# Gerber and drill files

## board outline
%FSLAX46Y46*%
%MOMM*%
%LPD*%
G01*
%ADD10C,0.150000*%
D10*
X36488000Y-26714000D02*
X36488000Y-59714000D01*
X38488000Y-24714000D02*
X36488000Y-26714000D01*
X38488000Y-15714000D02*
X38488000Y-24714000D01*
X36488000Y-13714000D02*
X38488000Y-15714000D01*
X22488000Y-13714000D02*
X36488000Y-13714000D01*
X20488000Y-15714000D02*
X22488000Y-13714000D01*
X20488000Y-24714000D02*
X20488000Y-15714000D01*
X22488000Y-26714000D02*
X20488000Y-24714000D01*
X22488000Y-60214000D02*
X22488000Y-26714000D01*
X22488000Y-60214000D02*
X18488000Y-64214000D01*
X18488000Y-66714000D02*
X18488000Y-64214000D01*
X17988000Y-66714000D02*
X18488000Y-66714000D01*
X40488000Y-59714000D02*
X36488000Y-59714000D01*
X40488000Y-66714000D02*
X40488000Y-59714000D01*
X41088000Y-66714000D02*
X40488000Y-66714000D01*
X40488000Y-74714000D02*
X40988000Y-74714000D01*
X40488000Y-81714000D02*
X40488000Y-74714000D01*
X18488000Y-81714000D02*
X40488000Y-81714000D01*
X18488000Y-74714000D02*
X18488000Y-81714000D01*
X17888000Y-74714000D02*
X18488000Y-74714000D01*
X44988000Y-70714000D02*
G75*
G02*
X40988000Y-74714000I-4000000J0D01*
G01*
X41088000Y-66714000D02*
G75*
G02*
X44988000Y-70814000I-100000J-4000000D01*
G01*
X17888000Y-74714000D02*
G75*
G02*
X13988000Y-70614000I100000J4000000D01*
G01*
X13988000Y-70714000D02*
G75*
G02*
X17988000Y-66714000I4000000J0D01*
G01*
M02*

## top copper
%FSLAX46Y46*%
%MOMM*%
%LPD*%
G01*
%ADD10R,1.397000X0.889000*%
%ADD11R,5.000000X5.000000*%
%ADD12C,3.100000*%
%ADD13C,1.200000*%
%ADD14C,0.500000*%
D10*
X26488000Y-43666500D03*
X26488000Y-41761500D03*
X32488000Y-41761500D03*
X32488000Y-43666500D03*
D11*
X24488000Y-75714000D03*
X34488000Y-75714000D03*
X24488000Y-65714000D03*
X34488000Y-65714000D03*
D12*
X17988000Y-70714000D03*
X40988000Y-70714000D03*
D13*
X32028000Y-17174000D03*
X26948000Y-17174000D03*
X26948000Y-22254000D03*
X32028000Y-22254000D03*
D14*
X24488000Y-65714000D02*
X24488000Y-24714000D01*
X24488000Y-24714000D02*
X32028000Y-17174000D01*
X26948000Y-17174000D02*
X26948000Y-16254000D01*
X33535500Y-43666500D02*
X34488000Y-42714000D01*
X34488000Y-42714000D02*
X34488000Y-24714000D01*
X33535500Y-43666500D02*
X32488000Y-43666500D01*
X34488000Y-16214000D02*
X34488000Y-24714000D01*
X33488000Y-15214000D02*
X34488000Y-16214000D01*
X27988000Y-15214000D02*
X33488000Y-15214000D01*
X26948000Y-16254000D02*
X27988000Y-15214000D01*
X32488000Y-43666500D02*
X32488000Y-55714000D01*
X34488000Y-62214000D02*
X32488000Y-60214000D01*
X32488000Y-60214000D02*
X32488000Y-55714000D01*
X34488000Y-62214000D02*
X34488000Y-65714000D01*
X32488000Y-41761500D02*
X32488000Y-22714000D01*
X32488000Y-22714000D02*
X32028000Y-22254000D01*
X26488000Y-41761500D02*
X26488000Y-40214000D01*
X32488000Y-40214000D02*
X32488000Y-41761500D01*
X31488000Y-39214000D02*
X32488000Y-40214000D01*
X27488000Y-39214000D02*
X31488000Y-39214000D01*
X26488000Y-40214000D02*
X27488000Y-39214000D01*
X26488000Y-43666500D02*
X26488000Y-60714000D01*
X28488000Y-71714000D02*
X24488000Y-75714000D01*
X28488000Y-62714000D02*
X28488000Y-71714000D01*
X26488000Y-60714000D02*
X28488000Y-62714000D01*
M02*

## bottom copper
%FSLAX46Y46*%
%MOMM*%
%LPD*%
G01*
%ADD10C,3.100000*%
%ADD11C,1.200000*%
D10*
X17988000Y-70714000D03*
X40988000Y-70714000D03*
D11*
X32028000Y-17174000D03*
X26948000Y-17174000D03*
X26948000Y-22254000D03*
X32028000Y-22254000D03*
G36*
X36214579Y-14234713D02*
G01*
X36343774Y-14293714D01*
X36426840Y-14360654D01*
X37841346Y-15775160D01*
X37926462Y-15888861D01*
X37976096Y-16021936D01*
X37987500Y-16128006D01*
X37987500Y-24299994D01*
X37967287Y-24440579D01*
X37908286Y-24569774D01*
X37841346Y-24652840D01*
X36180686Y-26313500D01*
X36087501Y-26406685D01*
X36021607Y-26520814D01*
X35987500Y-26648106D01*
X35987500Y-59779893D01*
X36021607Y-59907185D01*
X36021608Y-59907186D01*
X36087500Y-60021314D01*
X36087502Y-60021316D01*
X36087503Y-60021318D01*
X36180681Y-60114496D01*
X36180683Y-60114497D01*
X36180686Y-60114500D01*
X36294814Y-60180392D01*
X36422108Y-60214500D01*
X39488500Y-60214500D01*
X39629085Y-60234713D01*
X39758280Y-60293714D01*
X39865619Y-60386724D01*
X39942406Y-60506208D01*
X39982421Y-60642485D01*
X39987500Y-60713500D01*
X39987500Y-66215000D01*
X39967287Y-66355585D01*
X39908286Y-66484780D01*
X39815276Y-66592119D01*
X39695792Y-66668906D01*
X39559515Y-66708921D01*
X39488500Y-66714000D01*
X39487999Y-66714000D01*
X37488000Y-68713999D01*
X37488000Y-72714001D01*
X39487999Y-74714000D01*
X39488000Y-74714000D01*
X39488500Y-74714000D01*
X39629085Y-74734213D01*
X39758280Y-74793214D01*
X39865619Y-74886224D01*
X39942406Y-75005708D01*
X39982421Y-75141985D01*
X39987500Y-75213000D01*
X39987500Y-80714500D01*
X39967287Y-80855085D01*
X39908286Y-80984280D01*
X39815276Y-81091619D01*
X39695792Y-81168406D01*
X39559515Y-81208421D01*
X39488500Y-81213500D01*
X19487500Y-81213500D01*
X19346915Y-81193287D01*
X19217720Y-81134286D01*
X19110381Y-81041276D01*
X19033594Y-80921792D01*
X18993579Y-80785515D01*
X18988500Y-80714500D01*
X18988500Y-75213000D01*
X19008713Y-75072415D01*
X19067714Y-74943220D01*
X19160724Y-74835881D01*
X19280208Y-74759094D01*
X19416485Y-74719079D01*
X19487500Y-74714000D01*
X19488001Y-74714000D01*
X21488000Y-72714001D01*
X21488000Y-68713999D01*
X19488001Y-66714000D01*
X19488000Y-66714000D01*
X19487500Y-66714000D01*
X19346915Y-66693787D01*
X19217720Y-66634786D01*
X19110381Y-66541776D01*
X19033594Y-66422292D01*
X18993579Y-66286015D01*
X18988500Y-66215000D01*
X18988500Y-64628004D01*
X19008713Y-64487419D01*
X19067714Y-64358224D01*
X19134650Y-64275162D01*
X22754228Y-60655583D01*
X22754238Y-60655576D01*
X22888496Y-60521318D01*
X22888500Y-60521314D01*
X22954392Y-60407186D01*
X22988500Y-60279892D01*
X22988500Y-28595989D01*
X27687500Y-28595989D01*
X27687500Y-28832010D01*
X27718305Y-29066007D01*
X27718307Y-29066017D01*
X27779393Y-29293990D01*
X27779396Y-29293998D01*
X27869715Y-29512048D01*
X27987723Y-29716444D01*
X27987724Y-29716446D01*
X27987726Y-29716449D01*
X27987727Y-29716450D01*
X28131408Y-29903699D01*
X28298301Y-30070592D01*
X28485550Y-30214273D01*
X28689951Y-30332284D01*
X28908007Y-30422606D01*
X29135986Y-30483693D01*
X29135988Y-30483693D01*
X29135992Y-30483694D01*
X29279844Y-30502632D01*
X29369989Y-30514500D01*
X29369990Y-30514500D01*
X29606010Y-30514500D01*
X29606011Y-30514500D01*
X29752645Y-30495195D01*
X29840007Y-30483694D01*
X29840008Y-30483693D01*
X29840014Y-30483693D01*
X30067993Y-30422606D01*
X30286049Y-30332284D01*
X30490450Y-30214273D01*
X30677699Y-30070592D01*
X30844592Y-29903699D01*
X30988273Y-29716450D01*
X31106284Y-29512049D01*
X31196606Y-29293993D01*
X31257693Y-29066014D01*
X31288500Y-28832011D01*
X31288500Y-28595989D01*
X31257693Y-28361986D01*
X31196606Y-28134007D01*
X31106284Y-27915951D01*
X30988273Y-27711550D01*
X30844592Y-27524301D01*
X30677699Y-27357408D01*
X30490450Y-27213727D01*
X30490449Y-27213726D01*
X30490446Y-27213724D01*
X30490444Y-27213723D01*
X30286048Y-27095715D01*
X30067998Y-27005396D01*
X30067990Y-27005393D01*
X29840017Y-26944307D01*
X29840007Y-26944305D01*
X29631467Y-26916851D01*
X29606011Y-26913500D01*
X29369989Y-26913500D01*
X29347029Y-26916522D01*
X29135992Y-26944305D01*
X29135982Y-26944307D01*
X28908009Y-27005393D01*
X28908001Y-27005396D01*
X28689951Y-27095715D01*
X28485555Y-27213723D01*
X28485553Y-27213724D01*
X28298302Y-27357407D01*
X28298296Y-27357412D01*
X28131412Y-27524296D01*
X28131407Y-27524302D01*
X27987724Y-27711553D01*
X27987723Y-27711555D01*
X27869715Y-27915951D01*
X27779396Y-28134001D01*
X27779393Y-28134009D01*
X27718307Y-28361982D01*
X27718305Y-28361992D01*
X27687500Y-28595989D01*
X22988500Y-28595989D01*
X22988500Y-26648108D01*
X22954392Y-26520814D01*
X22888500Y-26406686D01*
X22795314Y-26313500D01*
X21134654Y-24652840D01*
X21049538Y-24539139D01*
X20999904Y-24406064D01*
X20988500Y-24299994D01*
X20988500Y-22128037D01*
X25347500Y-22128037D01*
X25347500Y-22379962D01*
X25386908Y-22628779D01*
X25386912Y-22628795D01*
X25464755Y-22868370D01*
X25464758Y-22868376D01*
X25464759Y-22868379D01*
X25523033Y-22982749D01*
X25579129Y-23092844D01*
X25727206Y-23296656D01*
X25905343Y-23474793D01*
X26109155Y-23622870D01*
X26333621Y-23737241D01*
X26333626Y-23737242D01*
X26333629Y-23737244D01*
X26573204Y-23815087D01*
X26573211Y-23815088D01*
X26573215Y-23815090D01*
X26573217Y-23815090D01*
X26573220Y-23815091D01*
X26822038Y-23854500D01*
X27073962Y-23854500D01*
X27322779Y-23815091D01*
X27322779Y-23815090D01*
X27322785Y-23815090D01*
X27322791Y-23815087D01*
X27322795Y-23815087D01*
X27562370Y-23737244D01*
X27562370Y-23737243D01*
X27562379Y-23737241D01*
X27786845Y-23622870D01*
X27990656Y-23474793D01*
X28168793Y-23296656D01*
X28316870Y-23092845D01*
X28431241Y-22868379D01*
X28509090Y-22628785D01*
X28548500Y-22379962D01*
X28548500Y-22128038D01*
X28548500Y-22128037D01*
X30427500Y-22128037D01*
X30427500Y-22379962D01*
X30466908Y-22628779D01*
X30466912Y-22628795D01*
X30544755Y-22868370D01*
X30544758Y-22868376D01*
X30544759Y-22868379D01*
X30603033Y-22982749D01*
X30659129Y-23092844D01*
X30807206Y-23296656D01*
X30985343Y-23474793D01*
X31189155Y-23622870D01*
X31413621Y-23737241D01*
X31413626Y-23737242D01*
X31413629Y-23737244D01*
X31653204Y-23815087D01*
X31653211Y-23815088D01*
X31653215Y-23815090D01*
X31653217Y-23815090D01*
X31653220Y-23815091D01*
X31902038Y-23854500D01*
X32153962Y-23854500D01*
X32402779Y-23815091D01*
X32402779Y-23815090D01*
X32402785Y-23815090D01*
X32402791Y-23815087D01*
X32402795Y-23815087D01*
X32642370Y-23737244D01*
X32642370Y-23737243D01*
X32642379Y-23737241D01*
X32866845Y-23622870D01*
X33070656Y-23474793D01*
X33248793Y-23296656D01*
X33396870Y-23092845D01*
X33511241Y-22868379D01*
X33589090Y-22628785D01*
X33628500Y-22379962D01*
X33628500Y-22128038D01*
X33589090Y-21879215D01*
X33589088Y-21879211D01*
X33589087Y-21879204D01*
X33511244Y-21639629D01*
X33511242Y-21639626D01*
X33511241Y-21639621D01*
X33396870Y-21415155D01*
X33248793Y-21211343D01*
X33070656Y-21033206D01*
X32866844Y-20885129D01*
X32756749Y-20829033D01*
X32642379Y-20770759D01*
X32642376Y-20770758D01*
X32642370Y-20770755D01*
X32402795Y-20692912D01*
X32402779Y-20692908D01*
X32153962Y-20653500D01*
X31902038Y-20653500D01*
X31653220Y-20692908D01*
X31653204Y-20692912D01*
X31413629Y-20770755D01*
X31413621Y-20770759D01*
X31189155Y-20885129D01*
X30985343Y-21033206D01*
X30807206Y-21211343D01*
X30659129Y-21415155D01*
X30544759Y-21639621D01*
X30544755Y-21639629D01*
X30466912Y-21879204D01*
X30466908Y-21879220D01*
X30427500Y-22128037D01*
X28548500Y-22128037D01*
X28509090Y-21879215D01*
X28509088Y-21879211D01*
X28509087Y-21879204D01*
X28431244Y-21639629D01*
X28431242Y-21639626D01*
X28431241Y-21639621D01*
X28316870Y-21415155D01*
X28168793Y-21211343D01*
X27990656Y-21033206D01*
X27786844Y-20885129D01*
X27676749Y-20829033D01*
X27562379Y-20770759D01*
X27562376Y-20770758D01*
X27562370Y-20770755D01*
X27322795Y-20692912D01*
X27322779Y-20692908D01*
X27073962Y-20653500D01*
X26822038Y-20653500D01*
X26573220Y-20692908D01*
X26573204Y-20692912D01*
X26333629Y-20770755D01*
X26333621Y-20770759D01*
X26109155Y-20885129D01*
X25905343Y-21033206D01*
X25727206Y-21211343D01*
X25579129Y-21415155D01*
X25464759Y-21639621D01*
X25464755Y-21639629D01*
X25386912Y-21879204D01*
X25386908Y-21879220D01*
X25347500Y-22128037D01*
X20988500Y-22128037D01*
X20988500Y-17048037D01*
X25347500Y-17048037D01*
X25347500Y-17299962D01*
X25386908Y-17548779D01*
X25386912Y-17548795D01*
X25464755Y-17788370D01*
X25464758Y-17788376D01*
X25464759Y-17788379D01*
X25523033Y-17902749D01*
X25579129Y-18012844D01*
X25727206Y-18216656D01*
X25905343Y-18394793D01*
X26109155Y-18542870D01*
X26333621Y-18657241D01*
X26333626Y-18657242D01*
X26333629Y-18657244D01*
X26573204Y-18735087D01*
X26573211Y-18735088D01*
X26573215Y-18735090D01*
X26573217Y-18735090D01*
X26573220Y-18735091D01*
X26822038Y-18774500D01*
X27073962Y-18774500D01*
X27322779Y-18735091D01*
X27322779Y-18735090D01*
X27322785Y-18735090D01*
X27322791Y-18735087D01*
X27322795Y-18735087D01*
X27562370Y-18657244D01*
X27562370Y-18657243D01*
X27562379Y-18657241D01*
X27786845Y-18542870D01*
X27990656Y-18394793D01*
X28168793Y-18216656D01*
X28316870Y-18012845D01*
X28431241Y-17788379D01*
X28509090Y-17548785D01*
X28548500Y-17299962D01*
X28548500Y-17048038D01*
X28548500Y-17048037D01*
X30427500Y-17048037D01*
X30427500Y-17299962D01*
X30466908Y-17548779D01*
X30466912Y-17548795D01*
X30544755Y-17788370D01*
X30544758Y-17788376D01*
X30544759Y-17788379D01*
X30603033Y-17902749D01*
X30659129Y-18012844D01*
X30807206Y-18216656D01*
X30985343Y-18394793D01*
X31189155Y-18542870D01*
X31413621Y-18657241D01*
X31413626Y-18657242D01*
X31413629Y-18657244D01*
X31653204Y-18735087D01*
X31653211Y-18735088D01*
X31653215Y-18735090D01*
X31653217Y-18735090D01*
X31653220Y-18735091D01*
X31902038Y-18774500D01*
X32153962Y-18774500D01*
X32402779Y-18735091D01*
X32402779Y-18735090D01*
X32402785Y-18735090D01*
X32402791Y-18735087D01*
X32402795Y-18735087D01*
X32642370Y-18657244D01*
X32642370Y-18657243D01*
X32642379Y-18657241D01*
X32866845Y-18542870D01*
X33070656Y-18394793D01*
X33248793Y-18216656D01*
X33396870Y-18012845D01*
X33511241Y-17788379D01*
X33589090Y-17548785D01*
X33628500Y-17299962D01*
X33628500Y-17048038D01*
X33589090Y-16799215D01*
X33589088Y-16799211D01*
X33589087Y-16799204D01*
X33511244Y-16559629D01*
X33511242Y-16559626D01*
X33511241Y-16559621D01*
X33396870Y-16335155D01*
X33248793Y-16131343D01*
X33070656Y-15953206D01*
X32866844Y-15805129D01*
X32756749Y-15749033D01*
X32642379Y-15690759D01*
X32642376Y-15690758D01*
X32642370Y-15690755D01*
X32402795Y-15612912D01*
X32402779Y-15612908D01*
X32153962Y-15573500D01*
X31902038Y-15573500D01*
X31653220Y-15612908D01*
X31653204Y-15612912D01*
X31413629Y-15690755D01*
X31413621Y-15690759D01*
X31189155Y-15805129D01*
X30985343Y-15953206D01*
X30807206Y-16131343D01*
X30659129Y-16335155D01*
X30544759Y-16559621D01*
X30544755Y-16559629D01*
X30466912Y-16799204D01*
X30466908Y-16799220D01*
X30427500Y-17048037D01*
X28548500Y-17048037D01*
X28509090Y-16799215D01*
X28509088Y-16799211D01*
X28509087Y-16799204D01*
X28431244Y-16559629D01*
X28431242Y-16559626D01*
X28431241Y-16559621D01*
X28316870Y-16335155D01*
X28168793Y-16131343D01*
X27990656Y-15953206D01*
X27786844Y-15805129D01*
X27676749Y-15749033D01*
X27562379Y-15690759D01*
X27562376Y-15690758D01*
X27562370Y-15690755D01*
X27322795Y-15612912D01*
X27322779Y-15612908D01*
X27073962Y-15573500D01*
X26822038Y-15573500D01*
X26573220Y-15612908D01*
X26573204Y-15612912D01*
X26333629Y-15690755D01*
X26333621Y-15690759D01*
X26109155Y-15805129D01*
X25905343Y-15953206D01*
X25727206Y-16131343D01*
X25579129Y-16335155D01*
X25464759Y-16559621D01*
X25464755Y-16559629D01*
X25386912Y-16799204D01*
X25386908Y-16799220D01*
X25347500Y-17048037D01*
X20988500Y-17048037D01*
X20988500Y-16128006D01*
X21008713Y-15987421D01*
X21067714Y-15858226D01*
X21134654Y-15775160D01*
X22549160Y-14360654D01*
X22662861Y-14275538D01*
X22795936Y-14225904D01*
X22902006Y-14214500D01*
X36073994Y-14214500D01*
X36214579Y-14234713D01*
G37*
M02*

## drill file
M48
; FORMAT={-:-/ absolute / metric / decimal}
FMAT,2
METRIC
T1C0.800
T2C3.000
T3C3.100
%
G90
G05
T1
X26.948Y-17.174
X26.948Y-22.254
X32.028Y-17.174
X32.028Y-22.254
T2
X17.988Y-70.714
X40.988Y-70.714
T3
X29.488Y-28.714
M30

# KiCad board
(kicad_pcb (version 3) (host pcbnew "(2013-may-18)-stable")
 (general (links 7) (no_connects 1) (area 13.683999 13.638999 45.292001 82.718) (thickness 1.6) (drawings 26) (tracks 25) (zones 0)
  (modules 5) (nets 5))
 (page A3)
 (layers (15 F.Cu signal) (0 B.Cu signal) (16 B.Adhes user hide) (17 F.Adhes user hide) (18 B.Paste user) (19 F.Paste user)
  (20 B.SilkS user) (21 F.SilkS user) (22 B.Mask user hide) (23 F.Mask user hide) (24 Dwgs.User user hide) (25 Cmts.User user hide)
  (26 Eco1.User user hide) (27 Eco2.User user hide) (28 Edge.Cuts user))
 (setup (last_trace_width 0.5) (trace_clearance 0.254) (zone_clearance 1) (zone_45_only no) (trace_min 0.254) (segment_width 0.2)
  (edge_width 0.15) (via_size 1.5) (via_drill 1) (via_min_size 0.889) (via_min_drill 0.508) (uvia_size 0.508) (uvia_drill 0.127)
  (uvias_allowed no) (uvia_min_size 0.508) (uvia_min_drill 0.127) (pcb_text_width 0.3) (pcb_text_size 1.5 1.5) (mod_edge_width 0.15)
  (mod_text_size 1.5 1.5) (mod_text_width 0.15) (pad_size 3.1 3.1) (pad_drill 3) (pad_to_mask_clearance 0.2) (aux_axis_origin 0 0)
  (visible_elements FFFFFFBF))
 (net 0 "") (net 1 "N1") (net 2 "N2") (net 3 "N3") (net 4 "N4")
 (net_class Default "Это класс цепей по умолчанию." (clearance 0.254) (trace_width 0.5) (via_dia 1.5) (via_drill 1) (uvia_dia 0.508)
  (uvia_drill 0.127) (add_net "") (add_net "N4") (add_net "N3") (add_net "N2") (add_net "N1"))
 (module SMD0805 (layer F.Cu) (at 26.488 42.714 90)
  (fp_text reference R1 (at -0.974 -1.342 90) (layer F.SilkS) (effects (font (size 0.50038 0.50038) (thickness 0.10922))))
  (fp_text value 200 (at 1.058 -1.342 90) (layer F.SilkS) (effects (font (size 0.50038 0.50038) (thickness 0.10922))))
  (pad 1 smd rect (at -0.9525 0 90) (size 0.889 1.397) (layers F.Cu F.Paste F.Mask) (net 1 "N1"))
  (pad 2 smd rect (at 0.9525 0 90) (size 0.889 1.397) (layers F.Cu F.Paste F.Mask) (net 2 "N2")))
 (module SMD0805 (layer F.Cu) (at 32.488 42.714 270)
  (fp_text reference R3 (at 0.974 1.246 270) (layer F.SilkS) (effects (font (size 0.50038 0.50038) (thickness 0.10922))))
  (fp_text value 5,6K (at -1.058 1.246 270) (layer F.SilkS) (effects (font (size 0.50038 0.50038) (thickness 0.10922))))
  (pad 1 smd rect (at -0.9525 0 270) (size 0.889 1.397) (layers F.Cu F.Paste F.Mask) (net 2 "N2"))
  (pad 2 smd rect (at 0.9525 0 270) (size 0.889 1.397) (layers F.Cu F.Paste F.Mask) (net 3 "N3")))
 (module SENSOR (layer F.Cu) (at 17.988 82.214)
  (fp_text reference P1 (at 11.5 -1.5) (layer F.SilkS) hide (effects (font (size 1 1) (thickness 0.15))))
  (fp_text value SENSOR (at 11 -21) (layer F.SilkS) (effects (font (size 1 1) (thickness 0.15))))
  (pad 2 smd rect (at 6.5 -6.5) (size 5 5) (layers F.Cu F.Mask) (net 1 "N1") (solder_mask_margin 0.1))
  (pad 3 smd rect (at 16.5 -6.5) (size 5 5) (layers F.Cu F.Mask))
  (pad 1 smd rect (at 6.5 -16.5) (size 5 5) (layers F.Cu F.Mask) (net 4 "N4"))
  (pad 4 smd rect (at 16.5 -16.5) (size 5 5) (layers F.Cu F.Mask) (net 3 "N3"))
  (pad "" np_thru_hole circle (at 0 -11.5) (size 3.1 3.1) (drill 3) (layers *.Cu *.Mask F.SilkS))
  (pad "" np_thru_hole circle (at 23 -11.5) (size 3.1 3.1) (drill 3) (layers *.Cu *.Mask F.SilkS)))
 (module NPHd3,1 (layer F.Cu) (at 29.488 28.714)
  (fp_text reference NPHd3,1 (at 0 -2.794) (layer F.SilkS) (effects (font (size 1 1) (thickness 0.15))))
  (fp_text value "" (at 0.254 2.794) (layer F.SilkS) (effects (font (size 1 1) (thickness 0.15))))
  (pad "" np_thru_hole circle (at 0 0) (size 3.1 3.1) (drill 3.1) (layers *.Cu *.Mask F.SilkS)))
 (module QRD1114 (layer F.Cu) (at 29.488 19.714 90)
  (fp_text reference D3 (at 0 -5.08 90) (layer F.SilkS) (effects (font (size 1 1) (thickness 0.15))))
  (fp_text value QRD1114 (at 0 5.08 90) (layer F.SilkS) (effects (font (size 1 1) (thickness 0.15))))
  (pad 4 thru_hole circle (at 2.54 2.54 90) (size 1.2 1.2) (drill 0.8) (layers *.Cu *.Mask F.SilkS) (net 4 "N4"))
  (pad 3 thru_hole circle (at 2.54 -2.54 90) (size 1.2 1.2) (drill 0.8) (layers *.Cu *.Mask F.SilkS) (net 3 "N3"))
  (pad 2 thru_hole circle (at -2.54 -2.54 90) (size 1.2 1.2) (drill 0.8) (layers *.Cu *.Mask F.SilkS) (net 4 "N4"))
  (pad 1 thru_hole circle (at -2.54 2.54 90) (size 1.2 1.2) (drill 0.8) (layers *.Cu *.Mask F.SilkS) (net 2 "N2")))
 (gr_line (start 36.488 26.714) (end 36.488 59.714) (angle 90) (layer Edge.Cuts) (width 0.15))
 (gr_line (start 38.488 24.714) (end 36.488 26.714) (angle 90) (layer Edge.Cuts) (width 0.15))
 (gr_line (start 38.488 15.714) (end 38.488 24.714) (angle 90) (layer Edge.Cuts) (width 0.15))
 (gr_line (start 36.488 13.714) (end 38.488 15.714) (angle 90) (layer Edge.Cuts) (width 0.15))
 (gr_line (start 22.488 13.714) (end 36.488 13.714) (angle 90) (layer Edge.Cuts) (width 0.15))
 (gr_line (start 20.488 15.714) (end 22.488 13.714) (angle 90) (layer Edge.Cuts) (width 0.15))
 (gr_line (start 20.488 24.714) (end 20.488 15.714) (angle 90) (layer Edge.Cuts) (width 0.15))
 (gr_line (start 22.488 26.714) (end 20.488 24.714) (angle 90) (layer Edge.Cuts) (width 0.15))
 (gr_line (start 22.488 60.214) (end 22.488 26.714) (angle 90) (layer Edge.Cuts) (width 0.15))
 (gr_line (start 22.488 60.214) (end 18.488 64.214) (angle 90) (layer Edge.Cuts) (width 0.15))
 (gr_line (start 18.488 66.714) (end 18.488 64.214) (angle 90) (layer Edge.Cuts) (width 0.15))
 (gr_line (start 17.988 66.714) (end 18.488 66.714) (angle 90) (layer Edge.Cuts) (width 0.15))
 (gr_line (start 40.488 59.714) (end 36.488 59.714) (angle 90) (layer Edge.Cuts) (width 0.15))
 (gr_line (start 40.488 66.714) (end 40.488 59.714) (angle 90) (layer Edge.Cuts) (width 0.15))
 (gr_line (start 41.088 66.714) (end 40.488 66.714) (angle 90) (layer Edge.Cuts) (width 0.15))
 (gr_line (start 40.488 74.714) (end 40.988 74.714) (angle 90) (layer Edge.Cuts) (width 0.15))
 (gr_line (start 40.488 81.714) (end 40.488 74.714) (angle 90) (layer Edge.Cuts) (width 0.15))
 (gr_line (start 18.488 81.714) (end 40.488 81.714) (angle 90) (layer Edge.Cuts) (width 0.15))
 (gr_line (start 18.488 74.714) (end 18.488 81.714) (angle 90) (layer Edge.Cuts) (width 0.15))
 (gr_line (start 17.888 74.714) (end 18.488 74.714) (angle 90) (layer Edge.Cuts) (width 0.15))
 (gr_arc (start 40.988 70.714) (end 44.988 70.714) (angle 90) (layer Edge.Cuts) (width 0.15))
 (gr_arc (start 40.988 70.714) (end 41.088 66.714) (angle 90) (layer Edge.Cuts) (width 0.15))
 (gr_arc (start 17.988 70.714) (end 17.888 74.714) (angle 90) (layer Edge.Cuts) (width 0.15))
 (gr_arc (start 17.988 70.714) (end 13.988 70.714) (angle 90) (layer Edge.Cuts) (width 0.15))
 (segment (start 24.488 65.714) (end 24.488 24.714) (width 0.5) (layer F.Cu) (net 4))
 (segment (start 24.488 24.714) (end 32.028 17.174) (width 0.5) (layer F.Cu) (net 4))
 (segment (start 26.948 17.174) (end 26.948 16.254) (width 0.5) (layer F.Cu) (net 3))
 (segment (start 33.5355 43.6665) (end 34.488 42.714) (width 0.5) (layer F.Cu) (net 3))
 (segment (start 34.488 42.714) (end 34.488 24.714) (width 0.5) (layer F.Cu) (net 3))
 (segment (start 33.5355 43.6665) (end 32.488 43.6665) (width 0.5) (layer F.Cu) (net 3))
 (segment (start 34.488 16.214) (end 34.488 24.714) (width 0.5) (layer F.Cu) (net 3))
 (segment (start 33.488 15.214) (end 34.488 16.214) (width 0.5) (layer F.Cu) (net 3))
 (segment (start 27.988 15.214) (end 33.488 15.214) (width 0.5) (layer F.Cu) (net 3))
 (segment (start 26.948 16.254) (end 27.988 15.214) (width 0.5) (layer F.Cu) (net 3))
 (segment (start 32.488 43.6665) (end 32.488 55.714) (width 0.5) (layer F.Cu) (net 3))
 (segment (start 34.488 62.214) (end 32.488 60.214) (width 0.5) (layer F.Cu) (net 3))
 (segment (start 32.488 60.214) (end 32.488 55.714) (width 0.5) (layer F.Cu) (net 3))
 (segment (start 34.488 62.214) (end 34.488 65.714) (width 0.5) (layer F.Cu) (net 3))
 (segment (start 32.488 41.7615) (end 32.488 22.714) (width 0.5) (layer F.Cu) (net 2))
 (segment (start 32.488 22.714) (end 32.028 22.254) (width 0.5) (layer F.Cu) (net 2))
 (segment (start 26.488 41.7615) (end 26.488 40.214) (width 0.5) (layer F.Cu) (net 2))
 (segment (start 32.488 40.214) (end 32.488 41.7615) (width 0.5) (layer F.Cu) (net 2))
 (segment (start 31.488 39.214) (end 32.488 40.214) (width 0.5) (layer F.Cu) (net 2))
 (segment (start 27.488 39.214) (end 31.488 39.214) (width 0.5) (layer F.Cu) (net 2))
 (segment (start 26.488 40.214) (end 27.488 39.214) (width 0.5) (layer F.Cu) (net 2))
 (segment (start 26.488 43.6665) (end 26.488 60.714) (width 0.5) (layer F.Cu) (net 1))
 (segment (start 28.488 71.714) (end 24.488 75.714) (width 0.5) (layer F.Cu) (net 1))
 (segment (start 28.488 62.714) (end 28.488 71.714) (width 0.5) (layer F.Cu) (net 1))
 (segment (start 26.488 60.714) (end 28.488 62.714) (width 0.5) (layer F.Cu) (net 1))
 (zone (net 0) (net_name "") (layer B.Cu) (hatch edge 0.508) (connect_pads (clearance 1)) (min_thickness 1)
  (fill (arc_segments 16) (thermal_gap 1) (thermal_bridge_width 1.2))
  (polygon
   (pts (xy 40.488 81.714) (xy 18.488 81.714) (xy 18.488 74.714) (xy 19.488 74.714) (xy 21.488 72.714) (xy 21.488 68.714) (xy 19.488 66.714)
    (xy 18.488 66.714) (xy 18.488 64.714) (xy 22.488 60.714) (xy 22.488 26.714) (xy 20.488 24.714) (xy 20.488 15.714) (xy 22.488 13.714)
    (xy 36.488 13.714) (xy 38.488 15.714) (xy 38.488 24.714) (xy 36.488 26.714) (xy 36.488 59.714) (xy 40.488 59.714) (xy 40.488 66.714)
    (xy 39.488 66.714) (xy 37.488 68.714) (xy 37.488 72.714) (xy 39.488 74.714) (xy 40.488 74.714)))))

